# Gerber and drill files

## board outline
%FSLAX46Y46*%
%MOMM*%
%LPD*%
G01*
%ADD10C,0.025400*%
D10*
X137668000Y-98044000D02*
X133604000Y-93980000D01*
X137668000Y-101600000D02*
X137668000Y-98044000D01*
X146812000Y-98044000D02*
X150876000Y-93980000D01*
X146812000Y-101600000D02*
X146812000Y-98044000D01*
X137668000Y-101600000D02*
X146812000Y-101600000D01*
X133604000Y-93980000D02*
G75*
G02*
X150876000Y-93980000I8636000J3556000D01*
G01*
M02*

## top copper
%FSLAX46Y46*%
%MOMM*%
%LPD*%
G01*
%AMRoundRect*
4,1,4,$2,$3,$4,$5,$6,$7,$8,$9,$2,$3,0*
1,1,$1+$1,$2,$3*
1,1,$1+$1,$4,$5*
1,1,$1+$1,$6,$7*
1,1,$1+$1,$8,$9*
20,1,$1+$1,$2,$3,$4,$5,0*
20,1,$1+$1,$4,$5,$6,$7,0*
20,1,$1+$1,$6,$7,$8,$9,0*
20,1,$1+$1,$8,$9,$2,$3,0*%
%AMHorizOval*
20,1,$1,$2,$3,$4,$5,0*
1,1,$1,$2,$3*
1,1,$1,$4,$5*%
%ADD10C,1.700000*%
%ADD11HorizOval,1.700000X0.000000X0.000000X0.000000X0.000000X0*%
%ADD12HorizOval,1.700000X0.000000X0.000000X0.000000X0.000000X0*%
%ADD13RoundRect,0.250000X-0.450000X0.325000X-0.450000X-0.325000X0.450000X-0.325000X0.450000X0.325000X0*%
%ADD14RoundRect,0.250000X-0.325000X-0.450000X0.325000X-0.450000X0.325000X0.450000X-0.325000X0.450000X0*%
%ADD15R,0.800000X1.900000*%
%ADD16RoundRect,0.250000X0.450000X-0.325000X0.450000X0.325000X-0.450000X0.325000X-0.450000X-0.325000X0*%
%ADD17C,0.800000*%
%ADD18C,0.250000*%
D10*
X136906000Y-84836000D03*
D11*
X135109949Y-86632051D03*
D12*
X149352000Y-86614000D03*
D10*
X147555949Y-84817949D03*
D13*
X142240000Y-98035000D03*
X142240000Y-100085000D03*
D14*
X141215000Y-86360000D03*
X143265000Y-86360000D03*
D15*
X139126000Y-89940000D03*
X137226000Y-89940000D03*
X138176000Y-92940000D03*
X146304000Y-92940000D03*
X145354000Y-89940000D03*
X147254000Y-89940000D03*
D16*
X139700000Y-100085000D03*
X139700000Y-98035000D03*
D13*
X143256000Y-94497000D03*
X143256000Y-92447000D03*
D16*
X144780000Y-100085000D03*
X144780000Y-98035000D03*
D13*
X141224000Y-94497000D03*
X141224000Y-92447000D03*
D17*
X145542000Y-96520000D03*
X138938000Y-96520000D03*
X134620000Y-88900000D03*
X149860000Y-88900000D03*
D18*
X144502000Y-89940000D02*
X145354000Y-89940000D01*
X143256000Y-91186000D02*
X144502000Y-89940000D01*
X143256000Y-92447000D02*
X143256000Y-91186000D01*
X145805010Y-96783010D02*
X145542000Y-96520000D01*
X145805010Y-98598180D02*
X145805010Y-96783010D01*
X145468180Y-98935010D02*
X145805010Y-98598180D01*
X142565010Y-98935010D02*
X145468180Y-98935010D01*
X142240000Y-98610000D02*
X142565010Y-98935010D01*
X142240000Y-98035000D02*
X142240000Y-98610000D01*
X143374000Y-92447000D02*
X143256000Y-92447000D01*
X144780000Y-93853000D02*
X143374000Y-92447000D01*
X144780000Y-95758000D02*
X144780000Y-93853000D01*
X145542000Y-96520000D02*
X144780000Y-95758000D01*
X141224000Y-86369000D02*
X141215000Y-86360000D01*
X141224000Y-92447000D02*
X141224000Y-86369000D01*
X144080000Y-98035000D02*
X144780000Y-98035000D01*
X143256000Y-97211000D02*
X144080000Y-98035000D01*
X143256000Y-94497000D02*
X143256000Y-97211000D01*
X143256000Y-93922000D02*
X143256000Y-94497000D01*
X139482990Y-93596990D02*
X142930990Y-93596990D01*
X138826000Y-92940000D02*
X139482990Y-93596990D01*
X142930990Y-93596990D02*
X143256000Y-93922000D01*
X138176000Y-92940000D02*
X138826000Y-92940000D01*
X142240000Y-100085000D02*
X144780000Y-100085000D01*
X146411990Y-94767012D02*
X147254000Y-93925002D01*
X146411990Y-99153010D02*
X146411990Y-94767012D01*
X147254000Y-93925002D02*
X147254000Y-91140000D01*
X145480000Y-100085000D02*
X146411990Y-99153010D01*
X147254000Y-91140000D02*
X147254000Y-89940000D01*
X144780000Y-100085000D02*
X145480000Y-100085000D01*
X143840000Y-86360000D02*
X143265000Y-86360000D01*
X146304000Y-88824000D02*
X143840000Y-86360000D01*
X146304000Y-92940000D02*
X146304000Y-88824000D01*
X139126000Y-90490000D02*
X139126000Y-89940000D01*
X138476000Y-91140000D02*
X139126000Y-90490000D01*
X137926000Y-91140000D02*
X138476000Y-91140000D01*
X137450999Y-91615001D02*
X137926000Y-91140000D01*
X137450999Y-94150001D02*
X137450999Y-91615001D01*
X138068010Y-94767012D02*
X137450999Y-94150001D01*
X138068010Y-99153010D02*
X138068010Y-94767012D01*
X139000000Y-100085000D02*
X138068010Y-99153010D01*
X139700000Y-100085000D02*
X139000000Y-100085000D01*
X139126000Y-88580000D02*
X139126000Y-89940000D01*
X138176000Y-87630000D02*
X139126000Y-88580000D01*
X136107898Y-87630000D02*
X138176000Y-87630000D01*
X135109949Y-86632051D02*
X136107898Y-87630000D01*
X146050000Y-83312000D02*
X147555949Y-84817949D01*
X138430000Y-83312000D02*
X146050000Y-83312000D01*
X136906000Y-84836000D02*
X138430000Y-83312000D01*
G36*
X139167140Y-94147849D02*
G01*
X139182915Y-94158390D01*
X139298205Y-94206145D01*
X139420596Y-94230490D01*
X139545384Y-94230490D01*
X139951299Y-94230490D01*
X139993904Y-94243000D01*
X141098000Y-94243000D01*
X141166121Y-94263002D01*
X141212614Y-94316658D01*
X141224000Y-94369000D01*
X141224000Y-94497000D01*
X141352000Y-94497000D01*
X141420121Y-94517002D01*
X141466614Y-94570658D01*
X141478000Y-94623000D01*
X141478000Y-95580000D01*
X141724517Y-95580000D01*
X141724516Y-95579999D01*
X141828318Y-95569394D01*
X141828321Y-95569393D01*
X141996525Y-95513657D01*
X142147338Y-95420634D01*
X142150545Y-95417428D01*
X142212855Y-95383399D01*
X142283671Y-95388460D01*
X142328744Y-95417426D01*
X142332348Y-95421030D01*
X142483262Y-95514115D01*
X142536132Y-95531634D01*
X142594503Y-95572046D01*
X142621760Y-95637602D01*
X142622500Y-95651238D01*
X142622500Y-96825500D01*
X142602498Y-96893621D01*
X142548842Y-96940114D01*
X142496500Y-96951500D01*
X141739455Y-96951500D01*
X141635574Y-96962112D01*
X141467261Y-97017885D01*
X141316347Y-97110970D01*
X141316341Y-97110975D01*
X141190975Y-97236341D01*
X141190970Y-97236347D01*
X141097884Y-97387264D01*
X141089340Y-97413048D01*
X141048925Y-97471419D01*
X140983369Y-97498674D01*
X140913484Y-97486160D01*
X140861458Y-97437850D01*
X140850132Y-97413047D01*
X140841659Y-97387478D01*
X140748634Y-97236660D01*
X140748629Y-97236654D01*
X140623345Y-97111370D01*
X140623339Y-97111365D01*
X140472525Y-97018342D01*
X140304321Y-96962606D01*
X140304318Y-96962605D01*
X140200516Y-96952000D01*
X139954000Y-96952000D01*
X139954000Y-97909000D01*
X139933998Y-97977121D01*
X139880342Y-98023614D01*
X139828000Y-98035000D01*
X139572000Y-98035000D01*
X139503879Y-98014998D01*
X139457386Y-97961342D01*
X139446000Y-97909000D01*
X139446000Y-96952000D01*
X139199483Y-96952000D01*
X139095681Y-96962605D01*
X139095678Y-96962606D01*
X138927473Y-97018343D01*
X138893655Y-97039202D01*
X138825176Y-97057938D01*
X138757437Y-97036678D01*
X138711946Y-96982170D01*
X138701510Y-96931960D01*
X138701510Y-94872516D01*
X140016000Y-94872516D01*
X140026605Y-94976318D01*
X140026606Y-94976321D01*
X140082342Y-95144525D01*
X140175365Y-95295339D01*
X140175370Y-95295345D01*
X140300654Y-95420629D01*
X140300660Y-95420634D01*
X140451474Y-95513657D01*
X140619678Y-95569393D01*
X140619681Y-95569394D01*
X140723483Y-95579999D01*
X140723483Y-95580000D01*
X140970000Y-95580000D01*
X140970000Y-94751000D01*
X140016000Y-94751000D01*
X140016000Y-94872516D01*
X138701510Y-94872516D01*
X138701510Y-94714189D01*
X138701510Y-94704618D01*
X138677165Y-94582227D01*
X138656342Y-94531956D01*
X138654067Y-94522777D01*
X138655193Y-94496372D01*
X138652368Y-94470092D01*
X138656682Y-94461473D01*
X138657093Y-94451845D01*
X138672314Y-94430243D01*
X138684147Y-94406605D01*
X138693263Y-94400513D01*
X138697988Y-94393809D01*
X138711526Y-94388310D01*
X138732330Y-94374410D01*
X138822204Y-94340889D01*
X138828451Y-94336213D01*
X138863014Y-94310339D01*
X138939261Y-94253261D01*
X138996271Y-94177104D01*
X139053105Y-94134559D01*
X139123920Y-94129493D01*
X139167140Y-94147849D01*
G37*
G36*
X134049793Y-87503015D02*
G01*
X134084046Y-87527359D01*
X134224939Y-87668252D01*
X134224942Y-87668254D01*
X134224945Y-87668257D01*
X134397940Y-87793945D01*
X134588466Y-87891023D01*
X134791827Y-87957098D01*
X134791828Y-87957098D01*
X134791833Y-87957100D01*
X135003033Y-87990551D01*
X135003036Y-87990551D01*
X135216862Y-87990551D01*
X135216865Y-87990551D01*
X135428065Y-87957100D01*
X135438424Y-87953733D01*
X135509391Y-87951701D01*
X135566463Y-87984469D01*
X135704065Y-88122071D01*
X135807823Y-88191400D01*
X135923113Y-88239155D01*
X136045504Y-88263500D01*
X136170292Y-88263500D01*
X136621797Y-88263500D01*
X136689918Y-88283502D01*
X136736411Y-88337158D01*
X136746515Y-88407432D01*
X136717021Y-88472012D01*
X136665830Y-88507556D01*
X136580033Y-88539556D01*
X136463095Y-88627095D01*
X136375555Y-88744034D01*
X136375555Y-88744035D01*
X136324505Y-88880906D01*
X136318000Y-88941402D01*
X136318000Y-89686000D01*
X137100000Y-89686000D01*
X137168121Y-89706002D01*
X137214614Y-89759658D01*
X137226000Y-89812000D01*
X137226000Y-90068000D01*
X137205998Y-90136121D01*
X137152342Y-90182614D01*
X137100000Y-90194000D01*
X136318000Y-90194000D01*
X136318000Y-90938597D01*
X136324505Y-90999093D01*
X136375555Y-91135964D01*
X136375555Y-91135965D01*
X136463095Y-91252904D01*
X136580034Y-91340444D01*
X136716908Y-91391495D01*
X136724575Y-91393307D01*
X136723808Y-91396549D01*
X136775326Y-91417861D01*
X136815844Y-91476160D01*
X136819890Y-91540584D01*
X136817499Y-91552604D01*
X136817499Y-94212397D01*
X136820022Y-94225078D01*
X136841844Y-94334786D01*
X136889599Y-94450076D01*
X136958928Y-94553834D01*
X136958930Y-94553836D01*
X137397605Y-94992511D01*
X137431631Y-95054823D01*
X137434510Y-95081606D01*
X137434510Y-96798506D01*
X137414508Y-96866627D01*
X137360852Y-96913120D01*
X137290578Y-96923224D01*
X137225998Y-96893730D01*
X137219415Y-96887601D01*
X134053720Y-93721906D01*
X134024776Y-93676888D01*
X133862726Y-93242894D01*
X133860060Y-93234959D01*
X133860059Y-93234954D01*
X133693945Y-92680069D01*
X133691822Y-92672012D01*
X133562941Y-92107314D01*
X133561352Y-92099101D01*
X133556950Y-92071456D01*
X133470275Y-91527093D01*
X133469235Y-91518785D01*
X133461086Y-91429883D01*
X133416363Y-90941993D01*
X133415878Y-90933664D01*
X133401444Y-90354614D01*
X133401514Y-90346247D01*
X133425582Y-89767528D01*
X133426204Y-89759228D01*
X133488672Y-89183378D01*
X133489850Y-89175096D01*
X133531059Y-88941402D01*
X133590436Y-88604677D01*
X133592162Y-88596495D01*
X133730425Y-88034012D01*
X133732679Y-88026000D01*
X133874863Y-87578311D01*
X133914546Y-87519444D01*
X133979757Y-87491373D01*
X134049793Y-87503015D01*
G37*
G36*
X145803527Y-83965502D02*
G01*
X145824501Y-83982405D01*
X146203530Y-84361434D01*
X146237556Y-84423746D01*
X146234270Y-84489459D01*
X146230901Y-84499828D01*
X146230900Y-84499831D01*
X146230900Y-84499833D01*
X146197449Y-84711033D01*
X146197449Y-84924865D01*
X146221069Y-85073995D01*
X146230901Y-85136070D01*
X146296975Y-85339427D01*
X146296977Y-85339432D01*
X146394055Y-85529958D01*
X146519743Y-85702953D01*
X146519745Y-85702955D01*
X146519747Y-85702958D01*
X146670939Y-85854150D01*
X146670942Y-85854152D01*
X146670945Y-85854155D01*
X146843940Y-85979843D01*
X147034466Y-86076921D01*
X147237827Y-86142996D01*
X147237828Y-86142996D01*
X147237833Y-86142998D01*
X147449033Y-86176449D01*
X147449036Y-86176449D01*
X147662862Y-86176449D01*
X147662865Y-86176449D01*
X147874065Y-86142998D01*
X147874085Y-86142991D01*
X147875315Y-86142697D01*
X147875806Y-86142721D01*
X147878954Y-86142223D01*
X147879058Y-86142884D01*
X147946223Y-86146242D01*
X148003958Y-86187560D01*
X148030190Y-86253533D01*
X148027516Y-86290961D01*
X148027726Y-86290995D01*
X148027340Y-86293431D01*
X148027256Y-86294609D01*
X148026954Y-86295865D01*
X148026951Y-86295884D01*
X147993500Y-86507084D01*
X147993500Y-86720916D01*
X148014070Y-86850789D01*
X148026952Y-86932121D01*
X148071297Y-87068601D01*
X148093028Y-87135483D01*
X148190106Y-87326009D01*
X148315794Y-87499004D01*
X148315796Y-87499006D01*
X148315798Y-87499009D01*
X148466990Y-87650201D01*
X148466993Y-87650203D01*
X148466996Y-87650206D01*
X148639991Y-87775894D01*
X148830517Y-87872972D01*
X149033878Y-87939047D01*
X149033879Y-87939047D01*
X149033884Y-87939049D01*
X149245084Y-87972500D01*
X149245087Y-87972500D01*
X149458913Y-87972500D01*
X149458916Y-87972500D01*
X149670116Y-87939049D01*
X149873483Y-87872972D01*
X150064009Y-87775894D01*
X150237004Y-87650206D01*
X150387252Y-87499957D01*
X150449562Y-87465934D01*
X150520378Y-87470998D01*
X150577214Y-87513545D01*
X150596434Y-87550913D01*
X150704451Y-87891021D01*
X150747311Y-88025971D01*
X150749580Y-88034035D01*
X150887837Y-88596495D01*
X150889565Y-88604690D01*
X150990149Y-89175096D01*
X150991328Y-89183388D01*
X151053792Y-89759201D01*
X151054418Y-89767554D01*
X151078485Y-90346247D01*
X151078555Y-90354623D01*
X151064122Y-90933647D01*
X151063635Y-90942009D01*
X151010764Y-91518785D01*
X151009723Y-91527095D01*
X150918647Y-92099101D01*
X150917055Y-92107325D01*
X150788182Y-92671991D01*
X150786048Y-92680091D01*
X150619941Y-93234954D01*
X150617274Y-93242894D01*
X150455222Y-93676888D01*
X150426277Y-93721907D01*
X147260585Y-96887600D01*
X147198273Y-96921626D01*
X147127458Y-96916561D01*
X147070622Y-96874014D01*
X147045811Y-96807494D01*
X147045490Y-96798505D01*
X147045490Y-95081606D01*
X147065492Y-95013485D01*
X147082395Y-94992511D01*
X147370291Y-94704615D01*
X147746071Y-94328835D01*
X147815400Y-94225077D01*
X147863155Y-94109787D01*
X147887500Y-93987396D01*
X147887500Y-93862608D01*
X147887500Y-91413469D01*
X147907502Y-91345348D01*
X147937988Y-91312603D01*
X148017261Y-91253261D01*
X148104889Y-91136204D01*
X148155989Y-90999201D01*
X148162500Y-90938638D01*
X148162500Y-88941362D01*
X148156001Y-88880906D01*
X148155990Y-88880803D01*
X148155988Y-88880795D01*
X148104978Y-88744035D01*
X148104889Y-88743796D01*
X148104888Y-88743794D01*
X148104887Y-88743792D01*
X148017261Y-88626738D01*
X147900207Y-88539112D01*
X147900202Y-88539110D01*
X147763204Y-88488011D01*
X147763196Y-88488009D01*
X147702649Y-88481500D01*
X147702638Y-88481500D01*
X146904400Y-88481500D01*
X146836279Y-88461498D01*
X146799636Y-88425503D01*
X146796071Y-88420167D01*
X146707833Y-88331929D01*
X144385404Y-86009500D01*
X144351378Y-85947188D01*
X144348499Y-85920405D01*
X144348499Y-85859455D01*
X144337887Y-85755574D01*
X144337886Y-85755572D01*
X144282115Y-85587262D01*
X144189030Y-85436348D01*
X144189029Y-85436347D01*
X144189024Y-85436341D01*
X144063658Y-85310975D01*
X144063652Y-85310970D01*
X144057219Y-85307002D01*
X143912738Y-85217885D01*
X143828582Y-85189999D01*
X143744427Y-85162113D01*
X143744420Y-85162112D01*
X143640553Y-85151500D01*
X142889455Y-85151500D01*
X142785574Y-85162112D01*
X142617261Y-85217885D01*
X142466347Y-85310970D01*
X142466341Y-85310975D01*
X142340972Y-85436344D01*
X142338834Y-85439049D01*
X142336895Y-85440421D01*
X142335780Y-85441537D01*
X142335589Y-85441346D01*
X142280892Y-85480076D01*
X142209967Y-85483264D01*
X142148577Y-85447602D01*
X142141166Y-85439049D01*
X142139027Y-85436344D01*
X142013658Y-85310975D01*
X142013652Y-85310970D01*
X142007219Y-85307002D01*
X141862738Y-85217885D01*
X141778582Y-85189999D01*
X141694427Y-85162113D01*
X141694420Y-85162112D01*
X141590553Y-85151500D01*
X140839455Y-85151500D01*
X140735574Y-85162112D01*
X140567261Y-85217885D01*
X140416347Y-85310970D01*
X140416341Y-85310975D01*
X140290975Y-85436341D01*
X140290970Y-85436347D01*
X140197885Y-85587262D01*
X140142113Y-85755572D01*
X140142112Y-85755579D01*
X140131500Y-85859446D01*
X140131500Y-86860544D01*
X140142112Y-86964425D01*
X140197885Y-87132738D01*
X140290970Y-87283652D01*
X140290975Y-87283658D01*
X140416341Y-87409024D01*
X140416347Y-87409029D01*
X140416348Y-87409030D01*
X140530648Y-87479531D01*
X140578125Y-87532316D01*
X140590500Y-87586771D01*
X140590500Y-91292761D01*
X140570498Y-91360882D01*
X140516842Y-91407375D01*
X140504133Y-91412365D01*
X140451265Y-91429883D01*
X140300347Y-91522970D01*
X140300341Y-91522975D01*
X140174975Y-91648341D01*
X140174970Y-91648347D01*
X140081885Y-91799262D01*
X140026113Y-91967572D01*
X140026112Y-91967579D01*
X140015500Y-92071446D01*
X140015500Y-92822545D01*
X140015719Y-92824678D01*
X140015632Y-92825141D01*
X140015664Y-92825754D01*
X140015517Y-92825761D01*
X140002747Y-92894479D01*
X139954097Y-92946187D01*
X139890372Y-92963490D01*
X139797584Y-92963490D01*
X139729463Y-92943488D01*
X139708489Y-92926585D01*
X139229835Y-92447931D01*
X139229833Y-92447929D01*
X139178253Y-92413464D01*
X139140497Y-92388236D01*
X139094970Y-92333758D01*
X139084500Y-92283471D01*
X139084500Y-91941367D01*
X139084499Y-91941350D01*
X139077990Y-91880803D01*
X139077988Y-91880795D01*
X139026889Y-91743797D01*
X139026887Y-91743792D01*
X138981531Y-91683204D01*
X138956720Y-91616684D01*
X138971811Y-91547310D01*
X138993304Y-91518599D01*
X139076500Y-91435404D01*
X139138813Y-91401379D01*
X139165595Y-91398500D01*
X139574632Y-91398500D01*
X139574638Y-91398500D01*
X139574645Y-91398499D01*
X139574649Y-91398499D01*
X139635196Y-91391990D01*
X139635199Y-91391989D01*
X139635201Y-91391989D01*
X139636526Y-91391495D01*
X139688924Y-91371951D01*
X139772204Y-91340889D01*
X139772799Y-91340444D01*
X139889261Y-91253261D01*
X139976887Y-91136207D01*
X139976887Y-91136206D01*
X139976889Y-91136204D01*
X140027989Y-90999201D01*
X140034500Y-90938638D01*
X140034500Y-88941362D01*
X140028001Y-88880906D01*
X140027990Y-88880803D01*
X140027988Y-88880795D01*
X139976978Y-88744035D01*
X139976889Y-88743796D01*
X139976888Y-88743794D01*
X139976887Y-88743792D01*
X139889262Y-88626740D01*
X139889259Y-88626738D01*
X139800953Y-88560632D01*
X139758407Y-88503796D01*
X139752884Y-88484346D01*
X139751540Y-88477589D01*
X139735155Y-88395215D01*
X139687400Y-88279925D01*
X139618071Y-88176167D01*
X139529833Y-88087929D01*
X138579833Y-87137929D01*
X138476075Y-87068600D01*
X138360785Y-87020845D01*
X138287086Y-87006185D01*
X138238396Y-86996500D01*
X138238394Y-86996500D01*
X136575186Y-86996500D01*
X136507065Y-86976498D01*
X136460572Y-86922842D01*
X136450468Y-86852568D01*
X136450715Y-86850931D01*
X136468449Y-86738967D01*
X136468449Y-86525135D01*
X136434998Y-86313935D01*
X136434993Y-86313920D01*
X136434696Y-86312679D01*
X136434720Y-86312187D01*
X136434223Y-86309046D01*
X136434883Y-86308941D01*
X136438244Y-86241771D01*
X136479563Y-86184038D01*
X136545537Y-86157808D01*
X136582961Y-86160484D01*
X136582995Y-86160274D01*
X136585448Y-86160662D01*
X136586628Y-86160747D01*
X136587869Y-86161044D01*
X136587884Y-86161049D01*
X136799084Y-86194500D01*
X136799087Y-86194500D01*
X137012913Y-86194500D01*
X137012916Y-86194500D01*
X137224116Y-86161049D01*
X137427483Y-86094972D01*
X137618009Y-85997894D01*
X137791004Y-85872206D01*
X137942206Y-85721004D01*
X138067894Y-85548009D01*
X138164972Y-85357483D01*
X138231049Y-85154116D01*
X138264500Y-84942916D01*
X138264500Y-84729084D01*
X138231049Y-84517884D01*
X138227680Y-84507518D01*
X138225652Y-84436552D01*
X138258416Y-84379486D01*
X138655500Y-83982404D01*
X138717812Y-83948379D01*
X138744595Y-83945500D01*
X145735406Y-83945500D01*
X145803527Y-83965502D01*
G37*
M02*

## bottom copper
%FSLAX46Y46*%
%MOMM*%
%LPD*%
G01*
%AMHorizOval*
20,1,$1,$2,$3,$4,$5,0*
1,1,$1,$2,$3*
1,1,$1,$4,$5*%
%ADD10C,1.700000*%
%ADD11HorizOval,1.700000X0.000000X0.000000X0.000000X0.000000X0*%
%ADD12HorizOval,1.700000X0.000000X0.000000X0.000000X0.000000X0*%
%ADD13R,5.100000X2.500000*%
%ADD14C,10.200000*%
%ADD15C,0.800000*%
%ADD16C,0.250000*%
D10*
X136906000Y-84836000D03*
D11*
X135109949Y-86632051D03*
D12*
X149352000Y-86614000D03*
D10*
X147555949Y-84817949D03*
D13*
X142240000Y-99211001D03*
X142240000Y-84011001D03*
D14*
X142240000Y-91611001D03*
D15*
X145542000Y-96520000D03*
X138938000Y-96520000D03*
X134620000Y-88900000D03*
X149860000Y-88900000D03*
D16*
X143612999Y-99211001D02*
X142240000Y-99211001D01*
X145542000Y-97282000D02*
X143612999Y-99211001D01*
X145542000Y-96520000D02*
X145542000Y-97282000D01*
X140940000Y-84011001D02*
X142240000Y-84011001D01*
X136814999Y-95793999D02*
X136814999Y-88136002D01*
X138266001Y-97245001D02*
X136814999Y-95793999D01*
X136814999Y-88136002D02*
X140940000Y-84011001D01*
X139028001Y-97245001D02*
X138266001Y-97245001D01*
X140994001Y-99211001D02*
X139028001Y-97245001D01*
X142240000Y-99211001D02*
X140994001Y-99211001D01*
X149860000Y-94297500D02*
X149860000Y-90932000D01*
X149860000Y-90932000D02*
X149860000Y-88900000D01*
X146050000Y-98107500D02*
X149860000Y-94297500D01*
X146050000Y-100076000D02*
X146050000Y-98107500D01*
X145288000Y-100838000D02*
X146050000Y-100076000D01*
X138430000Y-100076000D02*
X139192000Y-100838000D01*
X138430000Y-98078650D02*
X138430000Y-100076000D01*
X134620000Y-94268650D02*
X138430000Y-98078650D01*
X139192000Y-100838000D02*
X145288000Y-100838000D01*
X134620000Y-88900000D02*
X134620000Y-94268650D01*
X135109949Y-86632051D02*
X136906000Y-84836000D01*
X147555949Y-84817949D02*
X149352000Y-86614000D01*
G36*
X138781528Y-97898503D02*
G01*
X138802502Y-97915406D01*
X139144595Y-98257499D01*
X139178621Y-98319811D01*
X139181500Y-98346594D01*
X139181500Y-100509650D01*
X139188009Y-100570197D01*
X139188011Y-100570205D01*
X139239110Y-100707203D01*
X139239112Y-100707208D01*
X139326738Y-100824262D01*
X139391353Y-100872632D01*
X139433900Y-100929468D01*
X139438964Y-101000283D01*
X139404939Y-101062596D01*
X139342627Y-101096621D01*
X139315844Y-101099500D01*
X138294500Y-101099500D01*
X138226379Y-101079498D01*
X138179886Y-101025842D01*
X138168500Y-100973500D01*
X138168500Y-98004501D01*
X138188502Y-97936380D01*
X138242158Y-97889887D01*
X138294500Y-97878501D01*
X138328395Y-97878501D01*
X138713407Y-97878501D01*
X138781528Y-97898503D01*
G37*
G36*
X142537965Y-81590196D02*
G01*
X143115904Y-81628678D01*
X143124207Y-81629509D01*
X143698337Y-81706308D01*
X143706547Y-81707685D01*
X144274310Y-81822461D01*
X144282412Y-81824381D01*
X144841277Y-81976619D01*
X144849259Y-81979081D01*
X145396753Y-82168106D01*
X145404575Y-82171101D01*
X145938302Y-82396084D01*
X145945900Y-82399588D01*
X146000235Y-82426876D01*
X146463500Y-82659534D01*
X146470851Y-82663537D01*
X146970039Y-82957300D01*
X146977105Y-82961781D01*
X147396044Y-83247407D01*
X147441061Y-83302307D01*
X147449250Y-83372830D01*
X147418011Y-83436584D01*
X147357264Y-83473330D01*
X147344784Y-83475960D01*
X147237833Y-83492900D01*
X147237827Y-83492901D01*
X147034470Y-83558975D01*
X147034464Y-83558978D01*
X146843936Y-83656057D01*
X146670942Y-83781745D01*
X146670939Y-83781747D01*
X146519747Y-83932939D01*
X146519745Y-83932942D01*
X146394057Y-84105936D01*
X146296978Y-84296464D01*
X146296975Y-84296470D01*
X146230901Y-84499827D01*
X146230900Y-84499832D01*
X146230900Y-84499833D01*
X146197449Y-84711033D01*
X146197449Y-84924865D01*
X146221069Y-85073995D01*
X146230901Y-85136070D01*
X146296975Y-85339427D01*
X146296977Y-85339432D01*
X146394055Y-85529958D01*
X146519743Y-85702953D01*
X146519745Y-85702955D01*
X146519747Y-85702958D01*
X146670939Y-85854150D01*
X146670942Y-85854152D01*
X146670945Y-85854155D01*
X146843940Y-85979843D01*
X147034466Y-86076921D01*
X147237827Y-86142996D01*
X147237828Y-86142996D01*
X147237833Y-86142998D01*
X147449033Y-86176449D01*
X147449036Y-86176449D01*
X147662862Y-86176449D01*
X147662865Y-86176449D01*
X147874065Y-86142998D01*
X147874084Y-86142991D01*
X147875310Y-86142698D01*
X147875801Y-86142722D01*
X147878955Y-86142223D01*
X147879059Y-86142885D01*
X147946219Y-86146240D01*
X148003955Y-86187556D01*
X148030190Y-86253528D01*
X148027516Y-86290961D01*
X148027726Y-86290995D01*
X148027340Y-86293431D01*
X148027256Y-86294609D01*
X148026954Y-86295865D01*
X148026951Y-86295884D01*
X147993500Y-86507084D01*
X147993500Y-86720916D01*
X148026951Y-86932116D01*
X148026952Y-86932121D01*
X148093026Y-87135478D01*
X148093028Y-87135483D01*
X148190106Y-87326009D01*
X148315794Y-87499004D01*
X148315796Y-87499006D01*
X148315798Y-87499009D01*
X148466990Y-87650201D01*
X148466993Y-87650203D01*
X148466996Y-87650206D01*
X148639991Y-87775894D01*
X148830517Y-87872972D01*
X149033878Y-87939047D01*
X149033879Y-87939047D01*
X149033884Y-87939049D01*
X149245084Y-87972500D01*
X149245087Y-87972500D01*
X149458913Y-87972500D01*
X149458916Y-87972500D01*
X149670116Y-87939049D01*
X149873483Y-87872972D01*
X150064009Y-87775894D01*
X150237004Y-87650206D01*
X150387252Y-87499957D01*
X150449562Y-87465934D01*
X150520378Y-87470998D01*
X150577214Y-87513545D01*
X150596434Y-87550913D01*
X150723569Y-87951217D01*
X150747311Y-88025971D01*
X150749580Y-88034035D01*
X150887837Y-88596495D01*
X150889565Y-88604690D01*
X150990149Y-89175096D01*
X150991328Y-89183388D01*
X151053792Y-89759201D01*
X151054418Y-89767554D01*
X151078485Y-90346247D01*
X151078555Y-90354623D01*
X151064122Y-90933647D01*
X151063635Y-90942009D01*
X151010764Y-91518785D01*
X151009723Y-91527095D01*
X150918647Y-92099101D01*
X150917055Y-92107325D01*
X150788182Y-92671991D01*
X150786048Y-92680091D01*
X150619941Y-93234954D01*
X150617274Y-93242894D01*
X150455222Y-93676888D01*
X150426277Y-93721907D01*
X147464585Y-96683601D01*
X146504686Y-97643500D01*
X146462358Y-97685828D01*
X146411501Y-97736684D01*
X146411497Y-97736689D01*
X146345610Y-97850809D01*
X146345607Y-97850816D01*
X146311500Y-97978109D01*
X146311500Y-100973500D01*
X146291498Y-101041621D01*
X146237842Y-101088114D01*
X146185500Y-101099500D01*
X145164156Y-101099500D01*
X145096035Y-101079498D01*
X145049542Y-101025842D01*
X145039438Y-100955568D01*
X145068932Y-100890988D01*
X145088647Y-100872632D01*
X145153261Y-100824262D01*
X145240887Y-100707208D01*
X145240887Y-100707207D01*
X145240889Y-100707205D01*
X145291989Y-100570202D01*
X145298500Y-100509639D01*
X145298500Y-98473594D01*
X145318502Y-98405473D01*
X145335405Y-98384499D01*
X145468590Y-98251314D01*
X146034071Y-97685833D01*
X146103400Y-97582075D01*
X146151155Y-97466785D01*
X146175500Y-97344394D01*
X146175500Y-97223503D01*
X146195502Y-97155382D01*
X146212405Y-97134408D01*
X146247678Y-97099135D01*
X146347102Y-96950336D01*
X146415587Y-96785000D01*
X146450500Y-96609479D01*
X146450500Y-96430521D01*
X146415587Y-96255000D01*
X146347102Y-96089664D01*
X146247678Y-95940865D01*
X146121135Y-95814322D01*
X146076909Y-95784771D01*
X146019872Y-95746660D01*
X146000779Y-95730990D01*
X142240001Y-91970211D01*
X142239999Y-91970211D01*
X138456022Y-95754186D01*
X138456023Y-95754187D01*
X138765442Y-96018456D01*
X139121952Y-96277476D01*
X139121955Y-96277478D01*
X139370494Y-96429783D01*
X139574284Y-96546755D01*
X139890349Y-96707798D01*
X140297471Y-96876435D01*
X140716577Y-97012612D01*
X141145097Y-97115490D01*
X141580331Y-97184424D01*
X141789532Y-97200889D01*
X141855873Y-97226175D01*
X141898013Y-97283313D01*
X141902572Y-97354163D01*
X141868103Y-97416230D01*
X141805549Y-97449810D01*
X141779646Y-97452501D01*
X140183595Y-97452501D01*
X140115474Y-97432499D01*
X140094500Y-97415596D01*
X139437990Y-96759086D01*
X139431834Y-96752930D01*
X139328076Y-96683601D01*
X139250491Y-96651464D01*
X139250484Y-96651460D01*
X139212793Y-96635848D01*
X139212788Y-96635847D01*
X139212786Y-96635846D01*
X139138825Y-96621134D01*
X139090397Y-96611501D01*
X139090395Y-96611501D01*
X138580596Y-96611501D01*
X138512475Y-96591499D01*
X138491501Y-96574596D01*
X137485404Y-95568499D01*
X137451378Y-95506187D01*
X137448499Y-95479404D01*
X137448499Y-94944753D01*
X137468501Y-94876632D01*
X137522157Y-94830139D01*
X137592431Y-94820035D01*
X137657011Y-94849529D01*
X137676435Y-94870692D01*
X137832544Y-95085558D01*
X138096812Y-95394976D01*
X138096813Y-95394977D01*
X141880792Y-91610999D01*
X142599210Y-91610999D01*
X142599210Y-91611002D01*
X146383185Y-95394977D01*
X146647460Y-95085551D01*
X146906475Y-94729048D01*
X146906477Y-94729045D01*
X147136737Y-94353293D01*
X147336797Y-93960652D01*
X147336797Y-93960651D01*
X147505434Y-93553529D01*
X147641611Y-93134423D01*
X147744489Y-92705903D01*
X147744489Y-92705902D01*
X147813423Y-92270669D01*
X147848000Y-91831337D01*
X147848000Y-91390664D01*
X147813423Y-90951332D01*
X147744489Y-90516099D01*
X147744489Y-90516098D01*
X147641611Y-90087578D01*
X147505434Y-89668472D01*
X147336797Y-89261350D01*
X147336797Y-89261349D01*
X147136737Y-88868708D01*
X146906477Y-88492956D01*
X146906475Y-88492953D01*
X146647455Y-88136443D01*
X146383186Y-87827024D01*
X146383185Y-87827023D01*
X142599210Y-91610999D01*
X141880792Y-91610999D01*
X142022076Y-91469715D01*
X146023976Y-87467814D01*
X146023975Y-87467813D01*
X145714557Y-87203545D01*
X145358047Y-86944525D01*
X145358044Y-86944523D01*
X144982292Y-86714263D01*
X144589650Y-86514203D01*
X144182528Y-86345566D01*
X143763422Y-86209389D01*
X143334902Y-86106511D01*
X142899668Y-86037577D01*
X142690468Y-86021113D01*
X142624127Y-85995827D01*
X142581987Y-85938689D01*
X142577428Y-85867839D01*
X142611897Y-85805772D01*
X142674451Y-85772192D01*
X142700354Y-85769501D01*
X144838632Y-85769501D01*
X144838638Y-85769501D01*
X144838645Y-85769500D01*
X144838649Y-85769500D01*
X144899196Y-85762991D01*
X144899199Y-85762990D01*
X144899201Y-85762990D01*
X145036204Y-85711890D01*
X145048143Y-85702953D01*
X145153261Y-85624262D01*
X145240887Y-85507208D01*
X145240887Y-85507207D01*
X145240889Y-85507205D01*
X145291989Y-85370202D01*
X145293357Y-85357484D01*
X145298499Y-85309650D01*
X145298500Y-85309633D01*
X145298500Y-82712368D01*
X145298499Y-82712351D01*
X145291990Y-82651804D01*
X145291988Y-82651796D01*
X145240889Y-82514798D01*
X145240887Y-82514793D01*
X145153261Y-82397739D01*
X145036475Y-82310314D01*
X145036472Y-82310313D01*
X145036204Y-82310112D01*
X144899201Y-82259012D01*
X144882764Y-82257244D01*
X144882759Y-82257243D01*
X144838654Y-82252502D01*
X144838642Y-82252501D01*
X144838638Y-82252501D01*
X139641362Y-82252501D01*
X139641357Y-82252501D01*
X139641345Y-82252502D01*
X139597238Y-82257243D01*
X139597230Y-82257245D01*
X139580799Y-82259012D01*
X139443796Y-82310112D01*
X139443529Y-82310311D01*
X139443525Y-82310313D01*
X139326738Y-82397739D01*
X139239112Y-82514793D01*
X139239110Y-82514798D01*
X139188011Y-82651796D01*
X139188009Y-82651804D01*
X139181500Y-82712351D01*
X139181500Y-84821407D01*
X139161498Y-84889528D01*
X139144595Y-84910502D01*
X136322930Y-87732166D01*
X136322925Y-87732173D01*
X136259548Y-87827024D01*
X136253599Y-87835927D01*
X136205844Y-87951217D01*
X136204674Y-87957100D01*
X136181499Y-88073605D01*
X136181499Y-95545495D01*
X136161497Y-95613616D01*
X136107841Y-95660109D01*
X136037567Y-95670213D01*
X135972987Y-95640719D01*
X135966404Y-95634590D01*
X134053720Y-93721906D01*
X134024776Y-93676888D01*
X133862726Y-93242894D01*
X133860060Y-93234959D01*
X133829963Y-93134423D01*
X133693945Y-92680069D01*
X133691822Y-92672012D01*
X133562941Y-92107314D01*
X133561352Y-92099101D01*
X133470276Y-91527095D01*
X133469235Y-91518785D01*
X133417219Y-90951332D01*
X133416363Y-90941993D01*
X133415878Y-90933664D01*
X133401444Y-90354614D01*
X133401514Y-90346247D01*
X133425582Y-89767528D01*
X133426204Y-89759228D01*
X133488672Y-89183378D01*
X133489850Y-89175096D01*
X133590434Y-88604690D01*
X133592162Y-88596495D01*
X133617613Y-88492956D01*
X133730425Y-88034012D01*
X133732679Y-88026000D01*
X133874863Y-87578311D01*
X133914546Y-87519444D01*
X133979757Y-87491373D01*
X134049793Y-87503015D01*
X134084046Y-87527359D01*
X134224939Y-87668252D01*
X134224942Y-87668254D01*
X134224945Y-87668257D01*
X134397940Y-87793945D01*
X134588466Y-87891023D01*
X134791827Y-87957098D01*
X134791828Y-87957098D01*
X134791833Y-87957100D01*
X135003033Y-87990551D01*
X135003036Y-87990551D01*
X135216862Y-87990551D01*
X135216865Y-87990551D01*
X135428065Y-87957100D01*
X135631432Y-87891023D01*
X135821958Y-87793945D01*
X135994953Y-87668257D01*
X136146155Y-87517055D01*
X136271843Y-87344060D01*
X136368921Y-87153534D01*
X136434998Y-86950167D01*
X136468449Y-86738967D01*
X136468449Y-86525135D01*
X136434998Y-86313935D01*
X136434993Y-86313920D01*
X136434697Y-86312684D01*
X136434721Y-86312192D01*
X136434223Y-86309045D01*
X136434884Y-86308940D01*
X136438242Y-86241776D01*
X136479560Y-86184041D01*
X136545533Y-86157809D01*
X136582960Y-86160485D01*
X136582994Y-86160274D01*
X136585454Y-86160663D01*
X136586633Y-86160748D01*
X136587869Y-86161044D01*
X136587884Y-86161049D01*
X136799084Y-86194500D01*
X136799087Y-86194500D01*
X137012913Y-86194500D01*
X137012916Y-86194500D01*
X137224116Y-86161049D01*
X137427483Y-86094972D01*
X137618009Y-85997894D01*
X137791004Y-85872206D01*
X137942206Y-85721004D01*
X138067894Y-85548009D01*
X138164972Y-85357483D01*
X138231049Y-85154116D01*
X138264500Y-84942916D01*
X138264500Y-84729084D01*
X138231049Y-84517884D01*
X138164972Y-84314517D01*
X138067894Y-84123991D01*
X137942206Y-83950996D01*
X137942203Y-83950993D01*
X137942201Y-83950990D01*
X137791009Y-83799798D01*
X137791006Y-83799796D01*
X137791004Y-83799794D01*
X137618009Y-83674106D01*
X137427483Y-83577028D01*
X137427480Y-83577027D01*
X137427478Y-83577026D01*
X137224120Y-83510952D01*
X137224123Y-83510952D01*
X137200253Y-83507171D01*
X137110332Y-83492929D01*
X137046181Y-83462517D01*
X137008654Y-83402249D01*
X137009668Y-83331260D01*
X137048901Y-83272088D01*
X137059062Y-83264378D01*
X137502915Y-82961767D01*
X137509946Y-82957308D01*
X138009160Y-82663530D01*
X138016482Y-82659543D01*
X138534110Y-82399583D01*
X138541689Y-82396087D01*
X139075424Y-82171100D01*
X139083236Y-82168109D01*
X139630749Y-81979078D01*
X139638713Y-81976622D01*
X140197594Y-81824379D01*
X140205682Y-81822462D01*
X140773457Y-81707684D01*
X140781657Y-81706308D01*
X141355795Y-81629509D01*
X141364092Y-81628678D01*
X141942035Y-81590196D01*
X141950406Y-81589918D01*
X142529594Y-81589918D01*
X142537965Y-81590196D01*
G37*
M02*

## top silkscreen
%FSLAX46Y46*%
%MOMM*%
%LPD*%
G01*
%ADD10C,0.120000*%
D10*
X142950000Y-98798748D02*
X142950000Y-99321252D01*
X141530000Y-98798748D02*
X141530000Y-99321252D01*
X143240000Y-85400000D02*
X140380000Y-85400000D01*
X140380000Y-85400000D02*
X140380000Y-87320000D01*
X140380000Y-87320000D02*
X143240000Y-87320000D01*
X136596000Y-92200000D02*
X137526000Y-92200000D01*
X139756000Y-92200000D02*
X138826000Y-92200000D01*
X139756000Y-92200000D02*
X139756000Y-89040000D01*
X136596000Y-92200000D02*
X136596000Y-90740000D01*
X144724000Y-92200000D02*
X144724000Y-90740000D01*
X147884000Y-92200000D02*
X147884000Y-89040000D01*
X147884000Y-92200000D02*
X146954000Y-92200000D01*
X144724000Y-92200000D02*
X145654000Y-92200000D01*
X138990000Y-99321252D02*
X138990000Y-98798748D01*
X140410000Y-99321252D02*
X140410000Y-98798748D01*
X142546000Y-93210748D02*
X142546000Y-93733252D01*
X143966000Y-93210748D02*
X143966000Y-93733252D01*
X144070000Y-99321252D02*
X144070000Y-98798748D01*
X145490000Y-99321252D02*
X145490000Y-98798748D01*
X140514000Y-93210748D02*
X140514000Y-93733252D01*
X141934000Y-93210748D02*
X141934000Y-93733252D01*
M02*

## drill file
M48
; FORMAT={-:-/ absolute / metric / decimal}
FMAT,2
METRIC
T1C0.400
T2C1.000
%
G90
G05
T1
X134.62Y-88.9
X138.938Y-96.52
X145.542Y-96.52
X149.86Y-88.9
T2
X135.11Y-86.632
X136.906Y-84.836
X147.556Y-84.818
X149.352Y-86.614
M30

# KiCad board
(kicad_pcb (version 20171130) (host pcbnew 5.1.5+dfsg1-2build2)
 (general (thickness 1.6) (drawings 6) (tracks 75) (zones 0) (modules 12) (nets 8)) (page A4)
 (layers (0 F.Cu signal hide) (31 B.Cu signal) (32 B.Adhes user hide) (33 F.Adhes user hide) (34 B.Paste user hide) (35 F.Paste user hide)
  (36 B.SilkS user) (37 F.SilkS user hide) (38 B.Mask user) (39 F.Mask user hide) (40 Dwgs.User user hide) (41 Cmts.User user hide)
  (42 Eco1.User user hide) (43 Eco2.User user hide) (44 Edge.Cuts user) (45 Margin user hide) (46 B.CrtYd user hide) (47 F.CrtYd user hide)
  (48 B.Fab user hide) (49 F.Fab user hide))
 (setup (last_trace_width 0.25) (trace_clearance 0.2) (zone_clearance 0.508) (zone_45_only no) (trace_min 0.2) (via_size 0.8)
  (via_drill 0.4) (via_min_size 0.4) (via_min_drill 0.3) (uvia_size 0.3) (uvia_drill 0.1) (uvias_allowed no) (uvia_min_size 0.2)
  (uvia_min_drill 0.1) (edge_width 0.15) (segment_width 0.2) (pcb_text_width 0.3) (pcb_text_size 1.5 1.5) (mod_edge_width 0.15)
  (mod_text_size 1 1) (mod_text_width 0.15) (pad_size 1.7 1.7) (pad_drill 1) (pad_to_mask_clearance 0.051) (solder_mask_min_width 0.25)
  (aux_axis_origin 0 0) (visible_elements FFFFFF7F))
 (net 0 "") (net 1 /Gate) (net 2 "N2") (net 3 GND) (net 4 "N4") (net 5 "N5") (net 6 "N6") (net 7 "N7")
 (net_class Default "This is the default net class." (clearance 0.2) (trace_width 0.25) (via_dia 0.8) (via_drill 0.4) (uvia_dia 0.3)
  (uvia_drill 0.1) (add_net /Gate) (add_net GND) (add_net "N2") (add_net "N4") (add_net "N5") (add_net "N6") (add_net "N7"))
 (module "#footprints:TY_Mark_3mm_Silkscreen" (layer B.Cu) (at 148.844 91.44 180)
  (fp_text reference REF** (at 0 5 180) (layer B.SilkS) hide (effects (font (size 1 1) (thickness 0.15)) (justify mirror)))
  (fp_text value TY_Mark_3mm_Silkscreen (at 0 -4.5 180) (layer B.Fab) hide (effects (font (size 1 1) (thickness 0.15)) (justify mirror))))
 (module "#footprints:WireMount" (layer F.Cu) (at 136.906 84.836 315)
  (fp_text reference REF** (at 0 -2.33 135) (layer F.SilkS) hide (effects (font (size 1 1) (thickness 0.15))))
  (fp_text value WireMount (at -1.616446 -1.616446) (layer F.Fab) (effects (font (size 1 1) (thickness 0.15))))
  (pad 1 thru_hole circle (at 0 0 315) (size 1.7 1.7) (drill 1) (layers *.Cu *.Mask) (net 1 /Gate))
  (pad 2 thru_hole oval (at 0 2.54 315) (size 1.7 1.7) (drill 1) (layers *.Cu *.Mask) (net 1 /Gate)))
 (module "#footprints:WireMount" (layer F.Cu) (at 147.555949 84.817949 45)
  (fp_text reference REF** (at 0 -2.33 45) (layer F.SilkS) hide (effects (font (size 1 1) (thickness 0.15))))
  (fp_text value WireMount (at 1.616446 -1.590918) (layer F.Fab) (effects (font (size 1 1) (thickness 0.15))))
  (pad 2 thru_hole oval (at 0 2.54 45) (size 1.7 1.7) (drill 1) (layers *.Cu *.Mask) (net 1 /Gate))
  (pad 1 thru_hole circle (at 0 0 45) (size 1.7 1.7) (drill 1) (layers *.Cu *.Mask) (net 1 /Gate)))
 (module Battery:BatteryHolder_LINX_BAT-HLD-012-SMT (layer B.Cu) (at 142.24 91.611001 90)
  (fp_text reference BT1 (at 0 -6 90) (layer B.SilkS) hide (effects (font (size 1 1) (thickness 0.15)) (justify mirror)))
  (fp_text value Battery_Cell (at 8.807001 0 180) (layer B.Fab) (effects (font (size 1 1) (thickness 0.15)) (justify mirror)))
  (pad 1 smd rect (at -7.6 0 90) (size 2.5 5.1) (layers B.Cu B.Paste B.Mask) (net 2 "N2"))
  (pad 1 smd rect (at 7.6 0 90) (size 2.5 5.1) (layers B.Cu B.Paste B.Mask) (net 2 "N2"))
  (pad 2 smd circle (at 0 0 90) (size 10.2 10.2) (layers B.Cu B.Paste B.Mask) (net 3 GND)))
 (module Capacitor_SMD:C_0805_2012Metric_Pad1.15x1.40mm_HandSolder (layer F.Cu) (at 142.24 99.06 270)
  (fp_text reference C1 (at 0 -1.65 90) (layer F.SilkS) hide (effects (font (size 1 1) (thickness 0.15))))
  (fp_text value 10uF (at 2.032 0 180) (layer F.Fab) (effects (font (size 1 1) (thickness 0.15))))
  (fp_line (start -0.261252 -0.71) (end 0.261252 -0.71) (layer F.SilkS) (width 0.12))
  (fp_line (start -0.261252 0.71) (end 0.261252 0.71) (layer F.SilkS) (width 0.12))
  (pad 1 smd roundrect (at -1.025 0 270) (size 1.15 1.4) (layers F.Cu F.Paste F.Mask) (roundrect_rratio 0.217391) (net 2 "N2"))
  (pad 2 smd roundrect (at 1.025 0 270) (size 1.15 1.4) (layers F.Cu F.Paste F.Mask) (roundrect_rratio 0.217391) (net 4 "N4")))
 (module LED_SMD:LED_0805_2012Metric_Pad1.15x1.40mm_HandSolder (layer F.Cu) (at 142.24 86.36)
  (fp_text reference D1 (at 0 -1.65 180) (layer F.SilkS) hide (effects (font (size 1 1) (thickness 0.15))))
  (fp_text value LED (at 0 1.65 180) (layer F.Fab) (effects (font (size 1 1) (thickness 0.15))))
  (fp_line (start 1 -0.96) (end -1.86 -0.96) (layer F.SilkS) (width 0.12))
  (fp_line (start -1.86 -0.96) (end -1.86 0.96) (layer F.SilkS) (width 0.12))
  (fp_line (start -1.86 0.96) (end 1 0.96) (layer F.SilkS) (width 0.12))
  (pad 1 smd roundrect (at -1.025 0) (size 1.15 1.4) (layers F.Cu F.Paste F.Mask) (roundrect_rratio 0.217391) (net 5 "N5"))
  (pad 2 smd roundrect (at 1.025 0) (size 1.15 1.4) (layers F.Cu F.Paste F.Mask) (roundrect_rratio 0.217391) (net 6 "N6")))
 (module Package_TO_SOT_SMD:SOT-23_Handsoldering (layer F.Cu) (at 138.176 91.44 270)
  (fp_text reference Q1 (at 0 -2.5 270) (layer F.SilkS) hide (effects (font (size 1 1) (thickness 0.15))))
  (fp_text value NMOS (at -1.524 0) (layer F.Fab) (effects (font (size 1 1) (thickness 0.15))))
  (fp_line (start 0.76 1.58) (end 0.76 0.65) (layer F.SilkS) (width 0.12))
  (fp_line (start 0.76 -1.58) (end 0.76 -0.65) (layer F.SilkS) (width 0.12))
  (fp_line (start 0.76 -1.58) (end -2.4 -1.58) (layer F.SilkS) (width 0.12))
  (fp_line (start 0.76 1.58) (end -0.7 1.58) (layer F.SilkS) (width 0.12))
  (pad 1 smd rect (at -1.5 -0.95 270) (size 1.9 0.8) (layers F.Cu F.Paste F.Mask) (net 1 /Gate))
  (pad 2 smd rect (at -1.5 0.95 270) (size 1.9 0.8) (layers F.Cu F.Paste F.Mask) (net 3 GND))
  (pad 3 smd rect (at 1.5 0 270) (size 1.9 0.8) (layers F.Cu F.Paste F.Mask) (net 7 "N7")))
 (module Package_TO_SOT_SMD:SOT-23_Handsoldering (layer F.Cu) (at 146.304 91.44 270)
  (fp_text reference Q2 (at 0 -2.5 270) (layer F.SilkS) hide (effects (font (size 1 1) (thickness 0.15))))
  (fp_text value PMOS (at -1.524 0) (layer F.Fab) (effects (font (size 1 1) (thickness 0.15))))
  (fp_line (start 0.76 1.58) (end -0.7 1.58) (layer F.SilkS) (width 0.12))
  (fp_line (start 0.76 -1.58) (end -2.4 -1.58) (layer F.SilkS) (width 0.12))
  (fp_line (start 0.76 -1.58) (end 0.76 -0.65) (layer F.SilkS) (width 0.12))
  (fp_line (start 0.76 1.58) (end 0.76 0.65) (layer F.SilkS) (width 0.12))
  (pad 3 smd rect (at 1.5 0 270) (size 1.9 0.8) (layers F.Cu F.Paste F.Mask) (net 6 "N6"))
  (pad 2 smd rect (at -1.5 0.95 270) (size 1.9 0.8) (layers F.Cu F.Paste F.Mask) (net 2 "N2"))
  (pad 1 smd rect (at -1.5 -0.95 270) (size 1.9 0.8) (layers F.Cu F.Paste F.Mask) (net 4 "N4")))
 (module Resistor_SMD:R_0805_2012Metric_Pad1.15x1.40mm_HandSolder (layer F.Cu) (at 139.7 99.06 90)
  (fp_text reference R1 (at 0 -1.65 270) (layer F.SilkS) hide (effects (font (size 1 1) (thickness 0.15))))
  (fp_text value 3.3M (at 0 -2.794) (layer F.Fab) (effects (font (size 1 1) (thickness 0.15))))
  (fp_line (start -0.261252 -0.71) (end 0.261252 -0.71) (layer F.SilkS) (width 0.12))
  (fp_line (start -0.261252 0.71) (end 0.261252 0.71) (layer F.SilkS) (width 0.12))
  (pad 1 smd roundrect (at -1.025 0 90) (size 1.15 1.4) (layers F.Cu F.Paste F.Mask) (roundrect_rratio 0.217391) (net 1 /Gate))
  (pad 2 smd roundrect (at 1.025 0 90) (size 1.15 1.4) (layers F.Cu F.Paste F.Mask) (roundrect_rratio 0.217391) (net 3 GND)))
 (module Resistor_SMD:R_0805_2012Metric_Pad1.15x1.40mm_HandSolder (layer F.Cu) (at 143.256 93.472 270)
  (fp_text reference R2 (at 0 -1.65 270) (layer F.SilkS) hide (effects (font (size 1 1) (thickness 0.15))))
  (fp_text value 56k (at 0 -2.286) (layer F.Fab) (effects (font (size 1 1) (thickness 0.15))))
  (fp_line (start -0.261252 0.71) (end 0.261252 0.71) (layer F.SilkS) (width 0.12))
  (fp_line (start -0.261252 -0.71) (end 0.261252 -0.71) (layer F.SilkS) (width 0.12))
  (pad 2 smd roundrect (at 1.025 0 270) (size 1.15 1.4) (layers F.Cu F.Paste F.Mask) (roundrect_rratio 0.217391) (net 7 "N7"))
  (pad 1 smd roundrect (at -1.025 0 270) (size 1.15 1.4) (layers F.Cu F.Paste F.Mask) (roundrect_rratio 0.217391) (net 2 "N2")))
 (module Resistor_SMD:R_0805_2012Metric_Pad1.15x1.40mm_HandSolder (layer F.Cu) (at 144.78 99.06 90)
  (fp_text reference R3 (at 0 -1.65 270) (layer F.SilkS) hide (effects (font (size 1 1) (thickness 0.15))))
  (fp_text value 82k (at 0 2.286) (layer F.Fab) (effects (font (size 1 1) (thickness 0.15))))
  (fp_line (start -0.261252 -0.71) (end 0.261252 -0.71) (layer F.SilkS) (width 0.12))
  (fp_line (start -0.261252 0.71) (end 0.261252 0.71) (layer F.SilkS) (width 0.12))
  (pad 1 smd roundrect (at -1.025 0 90) (size 1.15 1.4) (layers F.Cu F.Paste F.Mask) (roundrect_rratio 0.217391) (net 4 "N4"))
  (pad 2 smd roundrect (at 1.025 0 90) (size 1.15 1.4) (layers F.Cu F.Paste F.Mask) (roundrect_rratio 0.217391) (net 7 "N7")))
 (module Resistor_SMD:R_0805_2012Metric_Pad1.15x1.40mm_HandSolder (layer F.Cu) (at 141.224 93.472 270)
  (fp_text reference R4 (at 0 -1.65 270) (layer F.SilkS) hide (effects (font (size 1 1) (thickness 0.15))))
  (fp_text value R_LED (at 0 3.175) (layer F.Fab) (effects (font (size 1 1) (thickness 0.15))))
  (fp_line (start -0.261252 0.71) (end 0.261252 0.71) (layer F.SilkS) (width 0.12))
  (fp_line (start -0.261252 -0.71) (end 0.261252 -0.71) (layer F.SilkS) (width 0.12))
  (pad 2 smd roundrect (at 1.025 0 270) (size 1.15 1.4) (layers F.Cu F.Paste F.Mask) (roundrect_rratio 0.217391) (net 3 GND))
  (pad 1 smd roundrect (at -1.025 0 270) (size 1.15 1.4) (layers F.Cu F.Paste F.Mask) (roundrect_rratio 0.217391) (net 5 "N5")))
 (gr_line (start 137.668 98.044) (end 133.604 93.98) (layer Edge.Cuts) (width 0.0254))
 (gr_line (start 137.668 101.6) (end 137.668 98.044) (layer Edge.Cuts) (width 0.0254))
 (gr_line (start 146.812 98.044) (end 150.876 93.98) (layer Edge.Cuts) (width 0.0254))
 (gr_line (start 146.812 101.6) (end 146.812 98.044) (layer Edge.Cuts) (width 0.0254))
 (gr_line (start 137.668 101.6) (end 146.812 101.6) (layer Edge.Cuts) (width 0.0254))
 (gr_arc (start 142.24 90.424) (end 150.876 93.98) (angle -224.7602701) (layer Edge.Cuts) (width 0.0254))
 (segment (start 144.502 89.94) (end 145.354 89.94) (width 0.25) (layer F.Cu) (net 2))
 (segment (start 143.256 91.186) (end 144.502 89.94) (width 0.25) (layer F.Cu) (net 2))
 (segment (start 143.256 92.447) (end 143.256 91.186) (width 0.25) (layer F.Cu) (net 2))
 (via (at 145.542 96.52) (size 0.8) (drill 0.4) (layers F.Cu B.Cu) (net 2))
 (segment (start 145.80501 96.78301) (end 145.542 96.52) (width 0.25) (layer F.Cu) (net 2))
 (segment (start 145.80501 98.59818) (end 145.80501 96.78301) (width 0.25) (layer F.Cu) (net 2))
 (segment (start 145.46818 98.93501) (end 145.80501 98.59818) (width 0.25) (layer F.Cu) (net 2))
 (segment (start 142.56501 98.93501) (end 145.46818 98.93501) (width 0.25) (layer F.Cu) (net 2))
 (segment (start 142.24 98.61) (end 142.56501 98.93501) (width 0.25) (layer F.Cu) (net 2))
 (segment (start 142.24 98.035) (end 142.24 98.61) (width 0.25) (layer F.Cu) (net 2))
 (segment (start 143.374 92.447) (end 143.256 92.447) (width 0.25) (layer F.Cu) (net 2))
 (segment (start 144.78 93.853) (end 143.374 92.447) (width 0.25) (layer F.Cu) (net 2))
 (segment (start 144.78 95.758) (end 144.78 93.853) (width 0.25) (layer F.Cu) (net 2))
 (segment (start 145.542 96.52) (end 144.78 95.758) (width 0.25) (layer F.Cu) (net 2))
 (segment (start 143.612999 99.211001) (end 142.24 99.211001) (width 0.25) (layer B.Cu) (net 2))
 (segment (start 145.542 97.282) (end 143.612999 99.211001) (width 0.25) (layer B.Cu) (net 2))
 (segment (start 145.542 96.52) (end 145.542 97.282) (width 0.25) (layer B.Cu) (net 2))
 (segment (start 140.94 84.011001) (end 142.24 84.011001) (width 0.25) (layer B.Cu) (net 2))
 (segment (start 136.814999 95.793999) (end 136.814999 88.136002) (width 0.25) (layer B.Cu) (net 2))
 (segment (start 138.266001 97.245001) (end 136.814999 95.793999) (width 0.25) (layer B.Cu) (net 2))
 (segment (start 136.814999 88.136002) (end 140.94 84.011001) (width 0.25) (layer B.Cu) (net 2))
 (segment (start 139.028001 97.245001) (end 138.266001 97.245001) (width 0.25) (layer B.Cu) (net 2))
 (segment (start 140.994001 99.211001) (end 139.028001 97.245001) (width 0.25) (layer B.Cu) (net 2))
 (segment (start 142.24 99.211001) (end 140.994001 99.211001) (width 0.25) (layer B.Cu) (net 2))
 (via (at 138.938 96.52) (size 0.8) (drill 0.4) (layers F.Cu B.Cu) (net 3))
 (via (at 134.62 88.9) (size 0.8) (drill 0.4) (layers F.Cu B.Cu) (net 3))
 (via (at 149.86 88.9) (size 0.8) (drill 0.4) (layers F.Cu B.Cu) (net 3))
 (segment (start 149.86 94.2975) (end 149.86 90.932) (width 0.25) (layer B.Cu) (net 3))
 (segment (start 149.86 90.932) (end 149.86 88.9) (width 0.25) (layer B.Cu) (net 3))
 (segment (start 146.05 98.1075) (end 149.86 94.2975) (width 0.25) (layer B.Cu) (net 3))
 (segment (start 146.05 100.076) (end 146.05 98.1075) (width 0.25) (layer B.Cu) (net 3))
 (segment (start 145.288 100.838) (end 146.05 100.076) (width 0.25) (layer B.Cu) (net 3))
 (segment (start 138.43 100.076) (end 139.192 100.838) (width 0.25) (layer B.Cu) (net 3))
 (segment (start 138.43 98.07865) (end 138.43 100.076) (width 0.25) (layer B.Cu) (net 3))
 (segment (start 134.62 94.26865) (end 138.43 98.07865) (width 0.25) (layer B.Cu) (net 3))
 (segment (start 139.192 100.838) (end 145.288 100.838) (width 0.25) (layer B.Cu) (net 3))
 (segment (start 134.62 88.9) (end 134.62 94.26865) (width 0.25) (layer B.Cu) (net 3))
 (segment (start 141.224 86.369) (end 141.215 86.36) (width 0.25) (layer F.Cu) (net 5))
 (segment (start 141.224 92.447) (end 141.224 86.369) (width 0.25) (layer F.Cu) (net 5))
 (segment (start 144.08 98.035) (end 144.78 98.035) (width 0.25) (layer F.Cu) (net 7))
 (segment (start 143.256 97.211) (end 144.08 98.035) (width 0.25) (layer F.Cu) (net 7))
 (segment (start 143.256 94.497) (end 143.256 97.211) (width 0.25) (layer F.Cu) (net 7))
 (segment (start 143.256 93.922) (end 143.256 94.497) (width 0.25) (layer F.Cu) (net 7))
 (segment (start 139.48299 93.59699) (end 142.93099 93.59699) (width 0.25) (layer F.Cu) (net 7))
 (segment (start 138.826 92.94) (end 139.48299 93.59699) (width 0.25) (layer F.Cu) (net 7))
 (segment (start 142.93099 93.59699) (end 143.256 93.922) (width 0.25) (layer F.Cu) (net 7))
 (segment (start 138.176 92.94) (end 138.826 92.94) (width 0.25) (layer F.Cu) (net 7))
 (segment (start 142.24 100.085) (end 144.78 100.085) (width 0.25) (layer F.Cu) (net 4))
 (segment (start 146.41199 94.767012) (end 147.254 93.925002) (width 0.25) (layer F.Cu) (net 4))
 (segment (start 146.41199 99.15301) (end 146.41199 94.767012) (width 0.25) (layer F.Cu) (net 4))
 (segment (start 147.254 93.925002) (end 147.254 91.14) (width 0.25) (layer F.Cu) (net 4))
 (segment (start 145.48 100.085) (end 146.41199 99.15301) (width 0.25) (layer F.Cu) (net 4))
 (segment (start 147.254 91.14) (end 147.254 89.94) (width 0.25) (layer F.Cu) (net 4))
 (segment (start 144.78 100.085) (end 145.48 100.085) (width 0.25) (layer F.Cu) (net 4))
 (segment (start 143.84 86.36) (end 143.265 86.36) (width 0.25) (layer F.Cu) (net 6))
 (segment (start 146.304 88.824) (end 143.84 86.36) (width 0.25) (layer F.Cu) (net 6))
 (segment (start 146.304 92.94) (end 146.304 88.824) (width 0.25) (layer F.Cu) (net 6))
 (segment (start 139.126 90.49) (end 139.126 89.94) (width 0.25) (layer F.Cu) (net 1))
 (segment (start 138.476 91.14) (end 139.126 90.49) (width 0.25) (layer F.Cu) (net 1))
 (segment (start 137.926 91.14) (end 138.476 91.14) (width 0.25) (layer F.Cu) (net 1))
 (segment (start 137.450999 91.615001) (end 137.926 91.14) (width 0.25) (layer F.Cu) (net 1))
 (segment (start 137.450999 94.150001) (end 137.450999 91.615001) (width 0.25) (layer F.Cu) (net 1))
 (segment (start 138.06801 94.767012) (end 137.450999 94.150001) (width 0.25) (layer F.Cu) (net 1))
 (segment (start 138.06801 99.15301) (end 138.06801 94.767012) (width 0.25) (layer F.Cu) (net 1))
 (segment (start 139 100.085) (end 138.06801 99.15301) (width 0.25) (layer F.Cu) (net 1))
 (segment (start 139.7 100.085) (end 139 100.085) (width 0.25) (layer F.Cu) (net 1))
 (segment (start 139.126 88.58) (end 139.126 89.94) (width 0.25) (layer F.Cu) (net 1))
 (segment (start 138.176 87.63) (end 139.126 88.58) (width 0.25) (layer F.Cu) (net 1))
 (segment (start 136.107898 87.63) (end 138.176 87.63) (width 0.25) (layer F.Cu) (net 1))
 (segment (start 135.109949 86.632051) (end 136.107898 87.63) (width 0.25) (layer F.Cu) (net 1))
 (segment (start 135.109949 86.632051) (end 136.906 84.836) (width 0.25) (layer B.Cu) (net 1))
 (segment (start 147.555949 84.817949) (end 149.352 86.614) (width 0.25) (layer B.Cu) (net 1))
 (segment (start 146.05 83.312) (end 147.555949 84.817949) (width 0.25) (layer F.Cu) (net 1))
 (segment (start 138.43 83.312) (end 146.05 83.312) (width 0.25) (layer F.Cu) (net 1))
 (segment (start 136.906 84.836) (end 138.43 83.312) (width 0.25) (layer F.Cu) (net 1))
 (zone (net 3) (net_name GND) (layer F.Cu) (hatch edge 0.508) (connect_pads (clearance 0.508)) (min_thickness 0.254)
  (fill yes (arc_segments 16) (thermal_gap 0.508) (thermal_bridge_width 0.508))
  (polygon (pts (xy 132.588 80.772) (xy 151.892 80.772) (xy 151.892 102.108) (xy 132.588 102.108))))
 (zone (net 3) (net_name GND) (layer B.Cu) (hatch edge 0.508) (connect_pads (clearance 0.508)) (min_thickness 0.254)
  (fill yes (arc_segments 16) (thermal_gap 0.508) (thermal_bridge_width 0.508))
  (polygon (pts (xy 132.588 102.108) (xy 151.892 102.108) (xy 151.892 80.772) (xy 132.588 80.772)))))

